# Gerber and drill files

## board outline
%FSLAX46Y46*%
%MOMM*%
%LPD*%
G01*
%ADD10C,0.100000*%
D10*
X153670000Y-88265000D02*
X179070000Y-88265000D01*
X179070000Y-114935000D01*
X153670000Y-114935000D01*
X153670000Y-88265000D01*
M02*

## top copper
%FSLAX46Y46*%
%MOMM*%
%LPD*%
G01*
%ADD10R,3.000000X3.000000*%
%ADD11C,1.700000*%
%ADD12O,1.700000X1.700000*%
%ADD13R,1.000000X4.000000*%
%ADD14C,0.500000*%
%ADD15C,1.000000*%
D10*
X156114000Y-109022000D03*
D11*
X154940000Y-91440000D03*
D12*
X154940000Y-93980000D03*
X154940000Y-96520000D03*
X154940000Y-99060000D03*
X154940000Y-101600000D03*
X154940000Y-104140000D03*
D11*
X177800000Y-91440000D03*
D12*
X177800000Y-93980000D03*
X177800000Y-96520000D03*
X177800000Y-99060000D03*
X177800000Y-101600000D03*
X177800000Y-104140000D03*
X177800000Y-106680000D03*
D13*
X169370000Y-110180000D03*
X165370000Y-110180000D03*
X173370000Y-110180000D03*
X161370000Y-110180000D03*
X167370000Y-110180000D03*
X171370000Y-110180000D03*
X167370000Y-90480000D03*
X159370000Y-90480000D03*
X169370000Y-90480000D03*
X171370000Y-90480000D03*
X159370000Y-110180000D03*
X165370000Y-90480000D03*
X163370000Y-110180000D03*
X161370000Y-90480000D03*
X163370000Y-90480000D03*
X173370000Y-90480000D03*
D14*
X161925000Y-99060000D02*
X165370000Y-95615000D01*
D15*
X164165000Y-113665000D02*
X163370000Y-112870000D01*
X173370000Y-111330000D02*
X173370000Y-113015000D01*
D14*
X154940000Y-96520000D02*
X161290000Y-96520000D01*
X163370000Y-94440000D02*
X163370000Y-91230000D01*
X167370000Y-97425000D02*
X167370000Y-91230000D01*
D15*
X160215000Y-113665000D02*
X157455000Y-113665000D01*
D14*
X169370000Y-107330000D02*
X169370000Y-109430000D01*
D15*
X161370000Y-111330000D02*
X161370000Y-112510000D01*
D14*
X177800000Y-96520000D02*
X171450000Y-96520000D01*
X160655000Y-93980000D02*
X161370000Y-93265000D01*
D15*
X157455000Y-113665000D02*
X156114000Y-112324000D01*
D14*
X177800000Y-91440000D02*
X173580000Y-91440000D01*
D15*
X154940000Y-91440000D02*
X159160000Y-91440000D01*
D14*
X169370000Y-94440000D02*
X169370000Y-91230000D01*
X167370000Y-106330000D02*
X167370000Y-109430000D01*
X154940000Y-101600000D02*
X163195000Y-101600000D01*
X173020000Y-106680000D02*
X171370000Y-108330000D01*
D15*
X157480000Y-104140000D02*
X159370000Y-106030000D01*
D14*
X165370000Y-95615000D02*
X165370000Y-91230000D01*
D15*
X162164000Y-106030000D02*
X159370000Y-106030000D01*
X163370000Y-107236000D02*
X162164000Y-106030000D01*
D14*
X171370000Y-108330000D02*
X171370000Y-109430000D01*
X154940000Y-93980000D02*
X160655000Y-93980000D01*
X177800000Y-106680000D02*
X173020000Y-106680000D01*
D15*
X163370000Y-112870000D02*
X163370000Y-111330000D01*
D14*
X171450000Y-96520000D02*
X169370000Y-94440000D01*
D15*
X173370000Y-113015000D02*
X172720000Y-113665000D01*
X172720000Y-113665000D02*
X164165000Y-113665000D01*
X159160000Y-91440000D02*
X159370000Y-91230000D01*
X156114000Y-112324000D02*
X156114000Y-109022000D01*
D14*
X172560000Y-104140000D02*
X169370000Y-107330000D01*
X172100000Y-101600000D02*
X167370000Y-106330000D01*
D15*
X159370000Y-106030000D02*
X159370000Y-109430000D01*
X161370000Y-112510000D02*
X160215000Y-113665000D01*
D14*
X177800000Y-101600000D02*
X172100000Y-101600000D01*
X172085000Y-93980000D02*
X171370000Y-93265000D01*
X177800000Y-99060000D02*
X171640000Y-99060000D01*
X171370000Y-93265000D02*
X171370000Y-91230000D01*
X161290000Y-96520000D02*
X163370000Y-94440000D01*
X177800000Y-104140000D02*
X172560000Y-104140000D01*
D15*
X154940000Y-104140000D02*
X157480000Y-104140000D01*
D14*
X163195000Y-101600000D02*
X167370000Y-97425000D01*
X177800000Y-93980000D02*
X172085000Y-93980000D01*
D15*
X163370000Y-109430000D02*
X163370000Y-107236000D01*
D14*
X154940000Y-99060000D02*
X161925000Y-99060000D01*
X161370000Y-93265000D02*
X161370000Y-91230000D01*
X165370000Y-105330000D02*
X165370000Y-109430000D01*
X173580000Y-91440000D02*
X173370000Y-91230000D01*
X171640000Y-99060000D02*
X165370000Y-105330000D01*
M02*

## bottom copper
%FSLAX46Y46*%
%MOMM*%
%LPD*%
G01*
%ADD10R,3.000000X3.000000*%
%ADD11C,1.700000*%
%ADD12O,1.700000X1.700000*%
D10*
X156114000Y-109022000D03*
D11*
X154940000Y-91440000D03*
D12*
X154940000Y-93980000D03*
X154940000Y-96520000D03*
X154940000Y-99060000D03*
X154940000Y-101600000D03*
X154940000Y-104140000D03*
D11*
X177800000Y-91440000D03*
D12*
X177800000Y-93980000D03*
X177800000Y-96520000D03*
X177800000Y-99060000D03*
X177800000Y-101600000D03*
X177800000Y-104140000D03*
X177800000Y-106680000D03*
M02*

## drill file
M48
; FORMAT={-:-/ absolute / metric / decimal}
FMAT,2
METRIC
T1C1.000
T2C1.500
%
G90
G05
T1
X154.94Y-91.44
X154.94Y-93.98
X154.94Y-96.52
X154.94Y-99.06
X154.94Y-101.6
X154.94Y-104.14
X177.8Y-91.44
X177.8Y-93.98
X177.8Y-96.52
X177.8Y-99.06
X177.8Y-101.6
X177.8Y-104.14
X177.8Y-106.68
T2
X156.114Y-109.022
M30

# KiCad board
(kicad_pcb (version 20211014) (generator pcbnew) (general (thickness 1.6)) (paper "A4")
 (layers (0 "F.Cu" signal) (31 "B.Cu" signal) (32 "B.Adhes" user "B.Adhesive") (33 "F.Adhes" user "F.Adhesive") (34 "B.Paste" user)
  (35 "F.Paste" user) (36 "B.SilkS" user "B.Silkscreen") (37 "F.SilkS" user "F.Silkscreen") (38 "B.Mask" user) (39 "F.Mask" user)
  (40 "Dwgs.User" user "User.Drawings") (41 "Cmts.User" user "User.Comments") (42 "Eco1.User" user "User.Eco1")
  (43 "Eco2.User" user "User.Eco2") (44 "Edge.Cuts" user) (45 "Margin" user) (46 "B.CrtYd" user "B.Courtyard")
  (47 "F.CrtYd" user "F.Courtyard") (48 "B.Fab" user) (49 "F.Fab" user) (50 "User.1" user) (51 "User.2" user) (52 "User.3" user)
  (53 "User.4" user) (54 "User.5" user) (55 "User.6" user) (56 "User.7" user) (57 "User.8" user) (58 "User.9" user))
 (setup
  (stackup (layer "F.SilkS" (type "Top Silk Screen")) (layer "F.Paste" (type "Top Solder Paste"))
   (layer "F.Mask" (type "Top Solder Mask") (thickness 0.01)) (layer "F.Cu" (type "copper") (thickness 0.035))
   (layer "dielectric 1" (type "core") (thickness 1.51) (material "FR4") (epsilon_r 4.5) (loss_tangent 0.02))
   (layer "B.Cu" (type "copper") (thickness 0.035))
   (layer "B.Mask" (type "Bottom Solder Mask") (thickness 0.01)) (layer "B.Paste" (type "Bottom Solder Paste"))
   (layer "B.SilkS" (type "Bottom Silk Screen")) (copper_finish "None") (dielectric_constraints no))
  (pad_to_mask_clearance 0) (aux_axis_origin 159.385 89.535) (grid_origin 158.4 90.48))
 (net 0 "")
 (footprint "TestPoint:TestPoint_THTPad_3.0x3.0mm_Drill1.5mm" (layer "F.Cu") (at 156.114 109.022)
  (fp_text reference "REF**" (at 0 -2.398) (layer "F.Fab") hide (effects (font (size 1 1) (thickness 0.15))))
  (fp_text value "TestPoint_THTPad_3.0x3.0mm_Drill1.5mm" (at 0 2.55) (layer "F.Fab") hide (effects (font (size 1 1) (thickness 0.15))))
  (pad "1" thru_hole rect (at 0 0) (size 3 3) (drill 1.5) (layers *.Cu *.Mask)))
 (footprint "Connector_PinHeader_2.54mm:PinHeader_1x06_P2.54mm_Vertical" (layer "F.Cu") (at 154.94 91.44)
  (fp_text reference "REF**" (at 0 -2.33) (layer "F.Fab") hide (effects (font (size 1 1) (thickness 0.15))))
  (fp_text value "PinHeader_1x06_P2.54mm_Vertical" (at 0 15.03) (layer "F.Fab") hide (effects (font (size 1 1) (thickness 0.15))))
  (pad "1" thru_hole circle (at 0 0) (size 1.7 1.7) (drill 1) (layers *.Cu *.Mask))
  (pad "2" thru_hole oval (at 0 2.54) (size 1.7 1.7) (drill 1) (layers *.Cu *.Mask))
  (pad "3" thru_hole oval (at 0 5.08) (size 1.7 1.7) (drill 1) (layers *.Cu *.Mask))
  (pad "4" thru_hole oval (at 0 7.62) (size 1.7 1.7) (drill 1) (layers *.Cu *.Mask))
  (pad "5" thru_hole oval (at 0 10.16) (size 1.7 1.7) (drill 1) (layers *.Cu *.Mask))
  (pad "6" thru_hole oval (at 0 12.7) (size 1.7 1.7) (drill 1) (layers *.Cu *.Mask)))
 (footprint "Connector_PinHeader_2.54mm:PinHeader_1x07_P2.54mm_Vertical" (layer "F.Cu") (at 177.8 91.44)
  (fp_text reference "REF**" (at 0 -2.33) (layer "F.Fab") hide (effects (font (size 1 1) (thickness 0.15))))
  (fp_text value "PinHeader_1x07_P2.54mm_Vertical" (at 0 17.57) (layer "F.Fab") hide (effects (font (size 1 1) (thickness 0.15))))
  (pad "1" thru_hole circle (at 0 0) (size 1.7 1.7) (drill 1) (layers *.Cu *.Mask))
  (pad "2" thru_hole oval (at 0 2.54) (size 1.7 1.7) (drill 1) (layers *.Cu *.Mask))
  (pad "3" thru_hole oval (at 0 5.08) (size 1.7 1.7) (drill 1) (layers *.Cu *.Mask))
  (pad "4" thru_hole oval (at 0 7.62) (size 1.7 1.7) (drill 1) (layers *.Cu *.Mask))
  (pad "5" thru_hole oval (at 0 10.16) (size 1.7 1.7) (drill 1) (layers *.Cu *.Mask))
  (pad "6" thru_hole oval (at 0 12.7) (size 1.7 1.7) (drill 1) (layers *.Cu *.Mask))
  (pad "7" thru_hole oval (at 0 15.24) (size 1.7 1.7) (drill 1) (layers *.Cu *.Mask)))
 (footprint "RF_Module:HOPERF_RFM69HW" (layer "F.Cu") (at 166.37 100.33 90)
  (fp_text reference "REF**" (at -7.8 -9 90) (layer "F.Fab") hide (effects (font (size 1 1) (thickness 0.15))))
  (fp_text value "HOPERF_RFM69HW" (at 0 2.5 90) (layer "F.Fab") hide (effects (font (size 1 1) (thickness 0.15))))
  (pad "" smd rect (at -9.85 3 90) (size 4 1) (layers "F.Cu" "F.Mask"))
  (pad "" smd rect (at -9.85 -1 90) (size 4 1) (layers "F.Cu" "F.Mask"))
  (pad "" smd rect (at -9.85 7 90) (size 4 1) (layers "F.Cu" "F.Mask"))
  (pad "" smd rect (at -9.85 -5 90) (size 4 1) (layers "F.Cu" "F.Mask"))
  (pad "" smd rect (at -9.85 1 90) (size 4 1) (layers "F.Cu" "F.Mask"))
  (pad "" smd rect (at -9.85 5 90) (size 4 1) (layers "F.Cu" "F.Mask"))
  (pad "" smd rect (at 9.85 1 90) (size 4 1) (layers "F.Cu" "F.Mask"))
  (pad "" smd rect (at 9.85 -7 90) (size 4 1) (layers "F.Cu" "F.Mask"))
  (pad "" smd rect (at 9.85 3 90) (size 4 1) (layers "F.Cu" "F.Mask"))
  (pad "" smd rect (at 9.85 5 90) (size 4 1) (layers "F.Cu" "F.Mask"))
  (pad "" smd rect (at -9.85 -7 90) (size 4 1) (layers "F.Cu" "F.Mask"))
  (pad "" smd rect (at 9.85 -1 90) (size 4 1) (layers "F.Cu" "F.Mask"))
  (pad "" smd rect (at -9.85 -3 90) (size 4 1) (layers "F.Cu" "F.Mask"))
  (pad "" smd rect (at 9.85 -5 90) (size 4 1) (layers "F.Cu" "F.Mask"))
  (pad "" smd rect (at 9.85 -3 90) (size 4 1) (layers "F.Cu" "F.Mask"))
  (pad "" smd rect (at 9.85 7 90) (size 4 1) (layers "F.Cu" "F.Mask")))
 (gr_rect (start 153.67 88.265) (end 179.07 114.935) (layer "Edge.Cuts") (width 0.1) (fill none))
 (segment (start 161.925 99.06) (end 165.37 95.615) (width 0.5) (layer "F.Cu") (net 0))
 (segment (start 164.165 113.665) (end 163.37 112.87) (width 1) (layer "F.Cu") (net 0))
 (segment (start 173.37 111.33) (end 173.37 113.015) (width 1) (layer "F.Cu") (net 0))
 (segment (start 154.94 96.52) (end 161.29 96.52) (width 0.5) (layer "F.Cu") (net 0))
 (segment (start 163.37 94.44) (end 163.37 91.23) (width 0.5) (layer "F.Cu") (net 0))
 (segment (start 167.37 97.425) (end 167.37 91.23) (width 0.5) (layer "F.Cu") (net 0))
 (segment (start 160.215 113.665) (end 157.455 113.665) (width 1) (layer "F.Cu") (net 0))
 (segment (start 169.37 107.33) (end 169.37 109.43) (width 0.5) (layer "F.Cu") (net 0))
 (segment (start 161.37 111.33) (end 161.37 112.51) (width 1) (layer "F.Cu") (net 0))
 (segment (start 177.8 96.52) (end 171.45 96.52) (width 0.5) (layer "F.Cu") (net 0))
 (segment (start 160.655 93.98) (end 161.37 93.265) (width 0.5) (layer "F.Cu") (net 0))
 (segment (start 157.455 113.665) (end 156.114 112.324) (width 1) (layer "F.Cu") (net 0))
 (segment (start 177.8 91.44) (end 173.58 91.44) (width 0.5) (layer "F.Cu") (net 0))
 (segment (start 154.94 91.44) (end 159.16 91.44) (width 1) (layer "F.Cu") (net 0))
 (segment (start 169.37 94.44) (end 169.37 91.23) (width 0.5) (layer "F.Cu") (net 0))
 (segment (start 167.37 106.33) (end 167.37 109.43) (width 0.5) (layer "F.Cu") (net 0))
 (segment (start 154.94 101.6) (end 163.195 101.6) (width 0.5) (layer "F.Cu") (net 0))
 (segment (start 173.02 106.68) (end 171.37 108.33) (width 0.5) (layer "F.Cu") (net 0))
 (segment (start 157.48 104.14) (end 159.37 106.03) (width 1) (layer "F.Cu") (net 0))
 (segment (start 165.37 95.615) (end 165.37 91.23) (width 0.5) (layer "F.Cu") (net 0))
 (segment (start 162.164 106.03) (end 159.37 106.03) (width 1) (layer "F.Cu") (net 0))
 (segment (start 163.37 107.236) (end 162.164 106.03) (width 1) (layer "F.Cu") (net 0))
 (segment (start 171.37 108.33) (end 171.37 109.43) (width 0.5) (layer "F.Cu") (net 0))
 (segment (start 154.94 93.98) (end 160.655 93.98) (width 0.5) (layer "F.Cu") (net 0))
 (segment (start 177.8 106.68) (end 173.02 106.68) (width 0.5) (layer "F.Cu") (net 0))
 (segment (start 163.37 112.87) (end 163.37 111.33) (width 1) (layer "F.Cu") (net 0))
 (segment (start 171.45 96.52) (end 169.37 94.44) (width 0.5) (layer "F.Cu") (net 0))
 (segment (start 173.37 113.015) (end 172.72 113.665) (width 1) (layer "F.Cu") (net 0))
 (segment (start 172.72 113.665) (end 164.165 113.665) (width 1) (layer "F.Cu") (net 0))
 (segment (start 159.16 91.44) (end 159.37 91.23) (width 1) (layer "F.Cu") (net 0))
 (segment (start 156.114 112.324) (end 156.114 109.022) (width 1) (layer "F.Cu") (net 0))
 (segment (start 172.56 104.14) (end 169.37 107.33) (width 0.5) (layer "F.Cu") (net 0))
 (segment (start 172.1 101.6) (end 167.37 106.33) (width 0.5) (layer "F.Cu") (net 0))
 (segment (start 159.37 106.03) (end 159.37 109.43) (width 1) (layer "F.Cu") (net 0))
 (segment (start 161.37 112.51) (end 160.215 113.665) (width 1) (layer "F.Cu") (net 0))
 (segment (start 177.8 101.6) (end 172.1 101.6) (width 0.5) (layer "F.Cu") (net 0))
 (segment (start 172.085 93.98) (end 171.37 93.265) (width 0.5) (layer "F.Cu") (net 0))
 (segment (start 177.8 99.06) (end 171.64 99.06) (width 0.5) (layer "F.Cu") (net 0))
 (segment (start 171.37 93.265) (end 171.37 91.23) (width 0.5) (layer "F.Cu") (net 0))
 (segment (start 161.29 96.52) (end 163.37 94.44) (width 0.5) (layer "F.Cu") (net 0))
 (segment (start 177.8 104.14) (end 172.56 104.14) (width 0.5) (layer "F.Cu") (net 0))
 (segment (start 154.94 104.14) (end 157.48 104.14) (width 1) (layer "F.Cu") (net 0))
 (segment (start 163.195 101.6) (end 167.37 97.425) (width 0.5) (layer "F.Cu") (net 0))
 (segment (start 177.8 93.98) (end 172.085 93.98) (width 0.5) (layer "F.Cu") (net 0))
 (segment (start 163.37 109.43) (end 163.37 107.236) (width 1) (layer "F.Cu") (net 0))
 (segment (start 154.94 99.06) (end 161.925 99.06) (width 0.5) (layer "F.Cu") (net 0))
 (segment (start 161.37 93.265) (end 161.37 91.23) (width 0.5) (layer "F.Cu") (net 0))
 (segment (start 165.37 105.33) (end 165.37 109.43) (width 0.5) (layer "F.Cu") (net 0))
 (segment (start 173.58 91.44) (end 173.37 91.23) (width 0.5) (layer "F.Cu") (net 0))
 (segment (start 171.64 99.06) (end 165.37 105.33) (width 0.5) (layer "F.Cu") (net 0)))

